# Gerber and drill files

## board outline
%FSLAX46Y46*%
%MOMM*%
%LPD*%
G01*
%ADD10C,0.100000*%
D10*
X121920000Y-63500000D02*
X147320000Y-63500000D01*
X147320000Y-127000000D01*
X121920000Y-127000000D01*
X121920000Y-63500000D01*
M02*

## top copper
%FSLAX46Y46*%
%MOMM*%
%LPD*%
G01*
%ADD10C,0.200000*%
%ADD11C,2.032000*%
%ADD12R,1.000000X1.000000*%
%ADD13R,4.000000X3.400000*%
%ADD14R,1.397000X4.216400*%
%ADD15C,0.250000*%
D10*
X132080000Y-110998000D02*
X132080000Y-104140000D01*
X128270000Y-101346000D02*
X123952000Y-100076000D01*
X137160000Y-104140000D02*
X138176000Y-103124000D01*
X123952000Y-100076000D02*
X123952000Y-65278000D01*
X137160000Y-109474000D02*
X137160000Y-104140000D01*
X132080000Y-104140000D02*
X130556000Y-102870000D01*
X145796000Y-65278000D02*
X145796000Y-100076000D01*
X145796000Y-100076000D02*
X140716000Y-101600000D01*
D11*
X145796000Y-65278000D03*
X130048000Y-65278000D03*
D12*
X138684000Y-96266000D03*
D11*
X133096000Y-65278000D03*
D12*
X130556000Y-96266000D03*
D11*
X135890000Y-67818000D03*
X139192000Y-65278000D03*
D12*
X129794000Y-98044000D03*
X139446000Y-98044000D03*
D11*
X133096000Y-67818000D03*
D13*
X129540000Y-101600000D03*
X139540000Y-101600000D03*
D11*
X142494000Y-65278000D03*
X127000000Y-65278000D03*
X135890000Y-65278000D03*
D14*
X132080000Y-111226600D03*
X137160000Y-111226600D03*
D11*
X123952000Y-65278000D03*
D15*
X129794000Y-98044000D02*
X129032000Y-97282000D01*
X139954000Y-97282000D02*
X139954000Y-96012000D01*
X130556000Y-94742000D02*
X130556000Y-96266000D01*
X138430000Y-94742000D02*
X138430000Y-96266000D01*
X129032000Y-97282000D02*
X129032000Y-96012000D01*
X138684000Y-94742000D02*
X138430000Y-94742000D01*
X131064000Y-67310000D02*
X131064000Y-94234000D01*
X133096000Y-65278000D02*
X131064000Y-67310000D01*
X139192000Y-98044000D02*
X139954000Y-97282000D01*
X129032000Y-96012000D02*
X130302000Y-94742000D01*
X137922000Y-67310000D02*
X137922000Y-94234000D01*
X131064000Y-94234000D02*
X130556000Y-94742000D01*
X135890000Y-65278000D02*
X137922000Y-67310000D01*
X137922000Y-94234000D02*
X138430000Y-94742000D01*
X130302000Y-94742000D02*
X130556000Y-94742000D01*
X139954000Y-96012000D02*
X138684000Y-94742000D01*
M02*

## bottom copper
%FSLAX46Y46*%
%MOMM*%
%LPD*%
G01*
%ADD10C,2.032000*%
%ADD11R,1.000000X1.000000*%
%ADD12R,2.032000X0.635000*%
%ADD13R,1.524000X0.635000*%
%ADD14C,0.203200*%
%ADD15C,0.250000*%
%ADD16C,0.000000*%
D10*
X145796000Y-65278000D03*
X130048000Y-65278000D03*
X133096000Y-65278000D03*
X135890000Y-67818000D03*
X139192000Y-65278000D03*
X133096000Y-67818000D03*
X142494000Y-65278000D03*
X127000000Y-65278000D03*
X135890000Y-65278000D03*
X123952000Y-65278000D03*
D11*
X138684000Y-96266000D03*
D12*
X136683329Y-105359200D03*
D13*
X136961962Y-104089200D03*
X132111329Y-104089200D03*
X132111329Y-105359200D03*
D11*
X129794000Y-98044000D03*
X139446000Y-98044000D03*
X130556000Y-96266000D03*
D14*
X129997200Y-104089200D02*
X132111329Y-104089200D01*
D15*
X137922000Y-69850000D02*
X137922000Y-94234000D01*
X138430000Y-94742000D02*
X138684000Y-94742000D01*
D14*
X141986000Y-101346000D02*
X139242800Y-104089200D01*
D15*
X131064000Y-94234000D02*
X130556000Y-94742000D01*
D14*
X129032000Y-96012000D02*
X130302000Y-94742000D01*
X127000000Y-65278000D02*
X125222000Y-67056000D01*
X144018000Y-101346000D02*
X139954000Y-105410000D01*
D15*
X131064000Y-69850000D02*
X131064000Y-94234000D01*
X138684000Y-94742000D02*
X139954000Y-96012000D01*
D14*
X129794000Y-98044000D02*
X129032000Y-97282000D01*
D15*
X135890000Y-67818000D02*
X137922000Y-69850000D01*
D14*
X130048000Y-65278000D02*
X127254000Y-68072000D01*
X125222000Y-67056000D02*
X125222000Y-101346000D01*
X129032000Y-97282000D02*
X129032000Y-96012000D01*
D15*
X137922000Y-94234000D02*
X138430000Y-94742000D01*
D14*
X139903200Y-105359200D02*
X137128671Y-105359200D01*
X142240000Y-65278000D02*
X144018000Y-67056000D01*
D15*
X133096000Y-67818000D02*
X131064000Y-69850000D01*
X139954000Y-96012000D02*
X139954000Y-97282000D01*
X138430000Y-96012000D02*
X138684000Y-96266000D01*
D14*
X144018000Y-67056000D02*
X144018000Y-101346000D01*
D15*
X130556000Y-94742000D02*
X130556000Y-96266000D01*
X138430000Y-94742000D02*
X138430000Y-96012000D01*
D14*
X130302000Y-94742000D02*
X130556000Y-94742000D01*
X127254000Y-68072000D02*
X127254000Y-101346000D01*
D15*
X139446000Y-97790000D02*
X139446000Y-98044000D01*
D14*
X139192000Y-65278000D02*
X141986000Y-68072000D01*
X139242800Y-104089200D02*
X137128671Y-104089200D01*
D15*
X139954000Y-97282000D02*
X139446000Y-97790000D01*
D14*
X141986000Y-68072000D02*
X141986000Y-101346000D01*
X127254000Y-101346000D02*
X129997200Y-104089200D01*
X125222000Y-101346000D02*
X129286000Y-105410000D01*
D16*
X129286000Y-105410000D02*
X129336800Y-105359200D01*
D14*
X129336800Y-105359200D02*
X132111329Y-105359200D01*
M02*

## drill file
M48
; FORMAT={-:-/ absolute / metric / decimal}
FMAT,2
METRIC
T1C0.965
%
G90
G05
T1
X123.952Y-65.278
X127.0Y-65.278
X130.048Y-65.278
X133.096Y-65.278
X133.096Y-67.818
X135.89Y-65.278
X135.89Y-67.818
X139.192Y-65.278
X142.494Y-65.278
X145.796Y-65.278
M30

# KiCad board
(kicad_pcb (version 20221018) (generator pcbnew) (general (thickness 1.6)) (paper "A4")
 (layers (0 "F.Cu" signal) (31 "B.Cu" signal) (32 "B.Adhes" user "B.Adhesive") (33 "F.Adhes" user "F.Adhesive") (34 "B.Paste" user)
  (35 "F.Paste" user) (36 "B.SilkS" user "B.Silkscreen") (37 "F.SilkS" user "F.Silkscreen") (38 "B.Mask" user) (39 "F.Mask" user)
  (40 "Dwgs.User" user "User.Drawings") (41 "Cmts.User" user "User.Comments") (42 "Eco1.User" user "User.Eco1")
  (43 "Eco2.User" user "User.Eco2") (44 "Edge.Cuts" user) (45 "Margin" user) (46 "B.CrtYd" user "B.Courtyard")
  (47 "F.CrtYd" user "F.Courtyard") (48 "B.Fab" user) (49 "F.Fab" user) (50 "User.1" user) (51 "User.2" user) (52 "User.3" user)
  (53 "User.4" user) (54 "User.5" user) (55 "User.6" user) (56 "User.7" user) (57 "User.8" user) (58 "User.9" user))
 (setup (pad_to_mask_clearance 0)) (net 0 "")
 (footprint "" (layer "F.Cu") (at 145.796 65.278)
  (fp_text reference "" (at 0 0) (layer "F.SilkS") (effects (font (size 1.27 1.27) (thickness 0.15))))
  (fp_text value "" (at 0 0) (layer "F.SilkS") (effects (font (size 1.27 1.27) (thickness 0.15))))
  (pad "1" thru_hole circle (at 0 0) (size 2.032 2.032) (drill 0.9652) (layers "*.Cu" "*.Mask")))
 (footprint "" (layer "F.Cu") (at 130.048 65.278)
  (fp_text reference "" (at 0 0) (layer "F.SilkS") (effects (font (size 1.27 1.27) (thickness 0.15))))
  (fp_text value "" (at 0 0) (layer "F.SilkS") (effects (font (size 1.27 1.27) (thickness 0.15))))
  (pad "1" thru_hole circle (at 0 0) (size 2.032 2.032) (drill 0.9652) (layers "*.Cu" "*.Mask")))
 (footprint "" (layer "F.Cu") (at 138.684 96.266)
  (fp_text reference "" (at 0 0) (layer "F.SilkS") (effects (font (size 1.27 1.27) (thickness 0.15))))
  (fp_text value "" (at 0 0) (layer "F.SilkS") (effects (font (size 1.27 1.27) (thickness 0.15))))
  (pad "1" smd rect (at 0 0) (size 1 1) (layers "F.Cu" "F.Mask")))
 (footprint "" (layer "F.Cu") (at 133.35 65.278)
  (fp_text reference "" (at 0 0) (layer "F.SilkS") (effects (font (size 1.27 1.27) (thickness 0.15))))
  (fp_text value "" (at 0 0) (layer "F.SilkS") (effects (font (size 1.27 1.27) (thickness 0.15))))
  (pad "1" thru_hole circle (at -0.254 0) (size 2.032 2.032) (drill 0.9652) (layers "*.Cu" "*.Mask")))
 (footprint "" (layer "F.Cu") (at 130.556 96.266)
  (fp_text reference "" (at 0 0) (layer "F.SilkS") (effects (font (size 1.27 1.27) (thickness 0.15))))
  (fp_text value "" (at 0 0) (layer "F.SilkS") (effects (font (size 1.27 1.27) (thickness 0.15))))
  (pad "1" smd rect (at 0 0) (size 1 1) (layers "F.Cu" "F.Mask")))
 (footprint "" (layer "F.Cu") (at 136.144 67.818)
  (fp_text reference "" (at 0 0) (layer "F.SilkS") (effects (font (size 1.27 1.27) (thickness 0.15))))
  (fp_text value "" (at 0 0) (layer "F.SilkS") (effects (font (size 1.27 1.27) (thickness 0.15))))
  (pad "1" thru_hole circle (at -0.254 0) (size 2.032 2.032) (drill 0.9652) (layers "*.Cu" "*.Mask")))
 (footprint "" (layer "F.Cu") (at 139.192 65.278)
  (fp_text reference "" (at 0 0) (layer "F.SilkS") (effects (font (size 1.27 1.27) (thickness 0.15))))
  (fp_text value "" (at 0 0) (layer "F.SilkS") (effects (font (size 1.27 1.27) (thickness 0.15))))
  (pad "1" thru_hole circle (at 0 0) (size 2.032 2.032) (drill 0.9652) (layers "*.Cu" "*.Mask")))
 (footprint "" (layer "F.Cu") (at 129.794 98.044)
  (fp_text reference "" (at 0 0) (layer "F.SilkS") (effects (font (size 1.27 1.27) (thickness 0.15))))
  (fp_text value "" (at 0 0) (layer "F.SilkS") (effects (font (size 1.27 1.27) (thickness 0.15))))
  (pad "1" smd rect (at 0 0) (size 1 1) (layers "F.Cu" "F.Mask")))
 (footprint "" (layer "F.Cu") (at 139.446 98.044)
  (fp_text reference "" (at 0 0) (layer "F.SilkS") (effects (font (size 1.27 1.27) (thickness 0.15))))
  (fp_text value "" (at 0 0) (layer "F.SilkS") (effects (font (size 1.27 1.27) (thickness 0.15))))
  (pad "1" smd rect (at 0 0) (size 1 1) (layers "F.Cu" "F.Mask")))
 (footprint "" (layer "F.Cu") (at 133.35 67.818)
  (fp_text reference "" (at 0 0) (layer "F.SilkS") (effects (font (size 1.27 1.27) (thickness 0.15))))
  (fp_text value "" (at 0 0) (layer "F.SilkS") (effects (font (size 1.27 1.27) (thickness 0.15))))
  (pad "1" thru_hole circle (at -0.254 0) (size 2.032 2.032) (drill 0.9652) (layers "*.Cu" "*.Mask")))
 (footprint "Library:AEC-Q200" (layer "F.Cu") (at 134.62 107.95)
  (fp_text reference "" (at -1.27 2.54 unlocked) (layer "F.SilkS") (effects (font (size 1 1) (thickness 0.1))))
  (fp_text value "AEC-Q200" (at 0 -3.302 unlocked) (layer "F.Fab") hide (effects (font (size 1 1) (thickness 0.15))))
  (pad "1" smd rect (at -5.08 -6.35 180) (size 4 3.4) (layers "F.Cu" "F.Mask"))
  (pad "2" smd rect (at 4.92 -6.35 180) (size 4 3.4) (layers "F.Cu" "F.Mask")))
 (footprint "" (layer "F.Cu") (at 142.494 65.278)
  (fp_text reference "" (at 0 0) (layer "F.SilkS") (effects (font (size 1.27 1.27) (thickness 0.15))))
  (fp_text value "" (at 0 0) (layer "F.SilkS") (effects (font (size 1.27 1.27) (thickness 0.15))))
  (pad "1" thru_hole circle (at 0 0) (size 2.032 2.032) (drill 0.9652) (layers "*.Cu" "*.Mask")))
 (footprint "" (layer "F.Cu") (at 127 65.278)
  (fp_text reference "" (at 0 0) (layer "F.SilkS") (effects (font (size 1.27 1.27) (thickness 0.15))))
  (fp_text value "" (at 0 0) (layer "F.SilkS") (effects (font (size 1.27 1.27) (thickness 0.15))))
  (pad "1" thru_hole circle (at 0 0) (size 2.032 2.032) (drill 0.9652) (layers "*.Cu" "*.Mask")))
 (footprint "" (layer "F.Cu") (at 136.144 65.278)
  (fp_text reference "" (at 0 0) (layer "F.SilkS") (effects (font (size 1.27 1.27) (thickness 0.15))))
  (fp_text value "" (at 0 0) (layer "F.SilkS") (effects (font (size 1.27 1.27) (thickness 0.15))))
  (pad "1" thru_hole circle (at -0.254 0) (size 2.032 2.032) (drill 0.9652) (layers "*.Cu" "*.Mask")))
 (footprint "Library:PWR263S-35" (layer "F.Cu") (at 135.89 112.268)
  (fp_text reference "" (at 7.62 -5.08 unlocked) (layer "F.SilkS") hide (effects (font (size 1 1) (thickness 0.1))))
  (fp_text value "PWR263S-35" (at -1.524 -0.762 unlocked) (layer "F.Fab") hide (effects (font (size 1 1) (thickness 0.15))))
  (pad "1" smd rect (at -3.81 -1.0414) (size 1.397 4.2164) (layers "F.Cu" "F.Mask"))
  (pad "2" smd rect (at 1.27 -1.0414) (size 1.397 4.2164) (layers "F.Cu" "F.Mask")))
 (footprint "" (layer "F.Cu") (at 123.952 65.278)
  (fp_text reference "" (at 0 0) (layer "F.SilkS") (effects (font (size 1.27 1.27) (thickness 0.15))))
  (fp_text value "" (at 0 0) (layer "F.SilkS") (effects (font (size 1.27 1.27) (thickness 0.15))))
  (pad "1" thru_hole circle (at 0 0) (size 2.032 2.032) (drill 0.9652) (layers "*.Cu" "*.Mask")))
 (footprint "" (layer "B.Cu") (at 138.684 96.266 180)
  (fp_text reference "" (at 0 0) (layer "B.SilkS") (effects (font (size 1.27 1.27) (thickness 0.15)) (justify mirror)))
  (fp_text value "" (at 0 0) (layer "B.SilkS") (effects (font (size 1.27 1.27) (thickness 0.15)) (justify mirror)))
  (pad "1" smd rect (at 0 0 180) (size 1 1) (layers "B.Cu" "B.Mask")))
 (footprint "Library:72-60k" (layer "B.Cu") (at 132.873329 109.1692 180)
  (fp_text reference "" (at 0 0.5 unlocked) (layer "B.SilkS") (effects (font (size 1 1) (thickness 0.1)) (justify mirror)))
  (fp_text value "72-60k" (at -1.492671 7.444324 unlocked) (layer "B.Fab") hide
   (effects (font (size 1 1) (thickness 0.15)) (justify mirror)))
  (pad "1" smd rect (at -3.81 3.81) (size 2.032 0.635) (layers "B.Cu" "B.Mask"))
  (pad "2" smd rect (at -4.088633 5.08) (size 1.524 0.635) (layers "B.Cu" "B.Mask"))
  (pad "3" smd rect (at 0.762 5.08) (size 1.524 0.635) (layers "B.Cu" "B.Mask"))
  (pad "4" smd rect (at 0.762 3.81) (size 1.524 0.635) (layers "B.Cu" "B.Mask")))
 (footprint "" (layer "B.Cu") (at 129.794 98.044 180)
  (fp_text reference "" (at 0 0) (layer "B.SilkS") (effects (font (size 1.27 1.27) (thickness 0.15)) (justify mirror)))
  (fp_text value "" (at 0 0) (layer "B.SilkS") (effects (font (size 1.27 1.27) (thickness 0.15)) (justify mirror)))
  (pad "1" smd rect (at 0 0 180) (size 1 1) (layers "B.Cu" "B.Mask")))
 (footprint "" (layer "B.Cu") (at 139.446 98.044 180)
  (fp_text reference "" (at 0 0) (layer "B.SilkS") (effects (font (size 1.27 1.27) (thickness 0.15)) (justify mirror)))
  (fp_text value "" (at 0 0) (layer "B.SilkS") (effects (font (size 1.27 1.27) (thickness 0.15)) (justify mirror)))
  (pad "1" smd rect (at 0 0 180) (size 1 1) (layers "B.Cu" "B.Mask")))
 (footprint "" (layer "B.Cu") (at 130.556 96.266 180)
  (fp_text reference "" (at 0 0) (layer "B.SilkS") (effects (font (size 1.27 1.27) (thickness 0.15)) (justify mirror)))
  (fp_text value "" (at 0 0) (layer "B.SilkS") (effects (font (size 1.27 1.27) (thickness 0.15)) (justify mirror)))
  (pad "1" smd rect (at 0 0 180) (size 1 1) (layers "B.Cu" "B.Mask")))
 (gr_line (start 132.08 110.998) (end 132.08 104.14) (stroke (width 0.2) (type default)) (layer "F.Cu"))
 (gr_line (start 128.27 101.346) (end 123.952 100.076) (stroke (width 0.2) (type default)) (layer "F.Cu"))
 (gr_line (start 137.16 104.14) (end 138.176 103.124) (stroke (width 0.2) (type default)) (layer "F.Cu"))
 (gr_line (start 123.952 100.076) (end 123.952 65.278) (stroke (width 0.2) (type default)) (layer "F.Cu"))
 (gr_line (start 137.16 109.474) (end 137.16 104.14) (stroke (width 0.2) (type default)) (layer "F.Cu"))
 (gr_line (start 132.08 104.14) (end 130.556 102.87) (stroke (width 0.2) (type default)) (layer "F.Cu"))
 (gr_line (start 145.796 65.278) (end 145.796 100.076) (stroke (width 0.2) (type default)) (layer "F.Cu"))
 (gr_line (start 145.796 100.076) (end 140.716 101.6) (stroke (width 0.2) (type default)) (layer "F.Cu"))
 (gr_rect (start 121.92 63.5) (end 147.32 127) (stroke (width 0.1) (type default)) (fill none) (layer "Edge.Cuts"))
 (segment (start 129.794 98.044) (end 129.032 97.282) (width 0.25) (layer "F.Cu") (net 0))
 (segment (start 139.954 97.282) (end 139.954 96.012) (width 0.25) (layer "F.Cu") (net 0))
 (segment (start 130.556 94.742) (end 130.556 96.266) (width 0.25) (layer "F.Cu") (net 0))
 (segment (start 138.43 94.742) (end 138.43 96.266) (width 0.25) (layer "F.Cu") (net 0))
 (segment (start 129.032 97.282) (end 129.032 96.012) (width 0.25) (layer "F.Cu") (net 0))
 (segment (start 138.684 94.742) (end 138.43 94.742) (width 0.25) (layer "F.Cu") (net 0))
 (segment (start 131.064 67.31) (end 131.064 94.234) (width 0.25) (layer "F.Cu") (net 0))
 (segment (start 133.096 65.278) (end 131.064 67.31) (width 0.25) (layer "F.Cu") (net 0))
 (segment (start 139.192 98.044) (end 139.954 97.282) (width 0.25) (layer "F.Cu") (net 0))
 (segment (start 129.032 96.012) (end 130.302 94.742) (width 0.25) (layer "F.Cu") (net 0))
 (segment (start 137.922 67.31) (end 137.922 94.234) (width 0.25) (layer "F.Cu") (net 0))
 (segment (start 131.064 94.234) (end 130.556 94.742) (width 0.25) (layer "F.Cu") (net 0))
 (segment (start 135.89 65.278) (end 137.922 67.31) (width 0.25) (layer "F.Cu") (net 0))
 (segment (start 137.922 94.234) (end 138.43 94.742) (width 0.25) (layer "F.Cu") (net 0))
 (segment (start 130.302 94.742) (end 130.556 94.742) (width 0.25) (layer "F.Cu") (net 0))
 (segment (start 139.954 96.012) (end 138.684 94.742) (width 0.25) (layer "F.Cu") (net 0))
 (segment (start 129.9972 104.0892) (end 132.111329 104.0892) (width 0.2032) (layer "B.Cu") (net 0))
 (segment (start 137.922 69.85) (end 137.922 94.234) (width 0.25) (layer "B.Cu") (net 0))
 (segment (start 138.43 94.742) (end 138.684 94.742) (width 0.25) (layer "B.Cu") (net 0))
 (segment (start 141.986 101.346) (end 139.2428 104.0892) (width 0.2032) (layer "B.Cu") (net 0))
 (segment (start 131.064 94.234) (end 130.556 94.742) (width 0.25) (layer "B.Cu") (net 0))
 (segment (start 129.032 96.012) (end 130.302 94.742) (width 0.2032) (layer "B.Cu") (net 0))
 (segment (start 127 65.278) (end 125.222 67.056) (width 0.2032) (layer "B.Cu") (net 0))
 (segment (start 144.018 101.346) (end 139.954 105.41) (width 0.2032) (layer "B.Cu") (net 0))
 (segment (start 131.064 69.85) (end 131.064 94.234) (width 0.25) (layer "B.Cu") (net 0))
 (segment (start 138.684 94.742) (end 139.954 96.012) (width 0.25) (layer "B.Cu") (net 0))
 (segment (start 129.794 98.044) (end 129.032 97.282) (width 0.2032) (layer "B.Cu") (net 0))
 (segment (start 135.89 67.818) (end 137.922 69.85) (width 0.25) (layer "B.Cu") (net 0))
 (segment (start 130.048 65.278) (end 127.254 68.072) (width 0.2032) (layer "B.Cu") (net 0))
 (segment (start 125.222 67.056) (end 125.222 101.346) (width 0.2032) (layer "B.Cu") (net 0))
 (segment (start 129.032 97.282) (end 129.032 96.012) (width 0.2032) (layer "B.Cu") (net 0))
 (segment (start 137.922 94.234) (end 138.43 94.742) (width 0.25) (layer "B.Cu") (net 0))
 (segment (start 139.9032 105.3592) (end 137.128671 105.3592) (width 0.2032) (layer "B.Cu") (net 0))
 (segment (start 142.24 65.278) (end 144.018 67.056) (width 0.2032) (layer "B.Cu") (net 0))
 (segment (start 133.096 67.818) (end 131.064 69.85) (width 0.25) (layer "B.Cu") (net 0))
 (segment (start 139.954 96.012) (end 139.954 97.282) (width 0.25) (layer "B.Cu") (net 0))
 (segment (start 138.43 96.012) (end 138.684 96.266) (width 0.25) (layer "B.Cu") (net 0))
 (segment (start 144.018 67.056) (end 144.018 101.346) (width 0.2032) (layer "B.Cu") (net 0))
 (segment (start 130.556 94.742) (end 130.556 96.266) (width 0.25) (layer "B.Cu") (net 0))
 (segment (start 138.43 94.742) (end 138.43 96.012) (width 0.25) (layer "B.Cu") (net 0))
 (segment (start 130.302 94.742) (end 130.556 94.742) (width 0.2032) (layer "B.Cu") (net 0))
 (segment (start 127.254 68.072) (end 127.254 101.346) (width 0.2032) (layer "B.Cu") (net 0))
 (segment (start 139.446 97.79) (end 139.446 98.044) (width 0.25) (layer "B.Cu") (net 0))
 (segment (start 139.192 65.278) (end 141.986 68.072) (width 0.2032) (layer "B.Cu") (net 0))
 (segment (start 139.2428 104.0892) (end 137.128671 104.0892) (width 0.2032) (layer "B.Cu") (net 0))
 (segment (start 139.954 97.282) (end 139.446 97.79) (width 0.25) (layer "B.Cu") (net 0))
 (segment (start 141.986 68.072) (end 141.986 101.346) (width 0.2032) (layer "B.Cu") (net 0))
 (segment (start 127.254 101.346) (end 129.9972 104.0892) (width 0.2032) (layer "B.Cu") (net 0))
 (segment (start 125.222 101.346) (end 129.286 105.41) (width 0.2032) (layer "B.Cu") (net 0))
 (segment (start 129.286 105.41) (end 129.3368 105.3592) (width 0) (layer "B.Cu") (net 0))
 (segment (start 129.3368 105.3592) (end 132.111329 105.3592) (width 0.2032) (layer "B.Cu") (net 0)))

